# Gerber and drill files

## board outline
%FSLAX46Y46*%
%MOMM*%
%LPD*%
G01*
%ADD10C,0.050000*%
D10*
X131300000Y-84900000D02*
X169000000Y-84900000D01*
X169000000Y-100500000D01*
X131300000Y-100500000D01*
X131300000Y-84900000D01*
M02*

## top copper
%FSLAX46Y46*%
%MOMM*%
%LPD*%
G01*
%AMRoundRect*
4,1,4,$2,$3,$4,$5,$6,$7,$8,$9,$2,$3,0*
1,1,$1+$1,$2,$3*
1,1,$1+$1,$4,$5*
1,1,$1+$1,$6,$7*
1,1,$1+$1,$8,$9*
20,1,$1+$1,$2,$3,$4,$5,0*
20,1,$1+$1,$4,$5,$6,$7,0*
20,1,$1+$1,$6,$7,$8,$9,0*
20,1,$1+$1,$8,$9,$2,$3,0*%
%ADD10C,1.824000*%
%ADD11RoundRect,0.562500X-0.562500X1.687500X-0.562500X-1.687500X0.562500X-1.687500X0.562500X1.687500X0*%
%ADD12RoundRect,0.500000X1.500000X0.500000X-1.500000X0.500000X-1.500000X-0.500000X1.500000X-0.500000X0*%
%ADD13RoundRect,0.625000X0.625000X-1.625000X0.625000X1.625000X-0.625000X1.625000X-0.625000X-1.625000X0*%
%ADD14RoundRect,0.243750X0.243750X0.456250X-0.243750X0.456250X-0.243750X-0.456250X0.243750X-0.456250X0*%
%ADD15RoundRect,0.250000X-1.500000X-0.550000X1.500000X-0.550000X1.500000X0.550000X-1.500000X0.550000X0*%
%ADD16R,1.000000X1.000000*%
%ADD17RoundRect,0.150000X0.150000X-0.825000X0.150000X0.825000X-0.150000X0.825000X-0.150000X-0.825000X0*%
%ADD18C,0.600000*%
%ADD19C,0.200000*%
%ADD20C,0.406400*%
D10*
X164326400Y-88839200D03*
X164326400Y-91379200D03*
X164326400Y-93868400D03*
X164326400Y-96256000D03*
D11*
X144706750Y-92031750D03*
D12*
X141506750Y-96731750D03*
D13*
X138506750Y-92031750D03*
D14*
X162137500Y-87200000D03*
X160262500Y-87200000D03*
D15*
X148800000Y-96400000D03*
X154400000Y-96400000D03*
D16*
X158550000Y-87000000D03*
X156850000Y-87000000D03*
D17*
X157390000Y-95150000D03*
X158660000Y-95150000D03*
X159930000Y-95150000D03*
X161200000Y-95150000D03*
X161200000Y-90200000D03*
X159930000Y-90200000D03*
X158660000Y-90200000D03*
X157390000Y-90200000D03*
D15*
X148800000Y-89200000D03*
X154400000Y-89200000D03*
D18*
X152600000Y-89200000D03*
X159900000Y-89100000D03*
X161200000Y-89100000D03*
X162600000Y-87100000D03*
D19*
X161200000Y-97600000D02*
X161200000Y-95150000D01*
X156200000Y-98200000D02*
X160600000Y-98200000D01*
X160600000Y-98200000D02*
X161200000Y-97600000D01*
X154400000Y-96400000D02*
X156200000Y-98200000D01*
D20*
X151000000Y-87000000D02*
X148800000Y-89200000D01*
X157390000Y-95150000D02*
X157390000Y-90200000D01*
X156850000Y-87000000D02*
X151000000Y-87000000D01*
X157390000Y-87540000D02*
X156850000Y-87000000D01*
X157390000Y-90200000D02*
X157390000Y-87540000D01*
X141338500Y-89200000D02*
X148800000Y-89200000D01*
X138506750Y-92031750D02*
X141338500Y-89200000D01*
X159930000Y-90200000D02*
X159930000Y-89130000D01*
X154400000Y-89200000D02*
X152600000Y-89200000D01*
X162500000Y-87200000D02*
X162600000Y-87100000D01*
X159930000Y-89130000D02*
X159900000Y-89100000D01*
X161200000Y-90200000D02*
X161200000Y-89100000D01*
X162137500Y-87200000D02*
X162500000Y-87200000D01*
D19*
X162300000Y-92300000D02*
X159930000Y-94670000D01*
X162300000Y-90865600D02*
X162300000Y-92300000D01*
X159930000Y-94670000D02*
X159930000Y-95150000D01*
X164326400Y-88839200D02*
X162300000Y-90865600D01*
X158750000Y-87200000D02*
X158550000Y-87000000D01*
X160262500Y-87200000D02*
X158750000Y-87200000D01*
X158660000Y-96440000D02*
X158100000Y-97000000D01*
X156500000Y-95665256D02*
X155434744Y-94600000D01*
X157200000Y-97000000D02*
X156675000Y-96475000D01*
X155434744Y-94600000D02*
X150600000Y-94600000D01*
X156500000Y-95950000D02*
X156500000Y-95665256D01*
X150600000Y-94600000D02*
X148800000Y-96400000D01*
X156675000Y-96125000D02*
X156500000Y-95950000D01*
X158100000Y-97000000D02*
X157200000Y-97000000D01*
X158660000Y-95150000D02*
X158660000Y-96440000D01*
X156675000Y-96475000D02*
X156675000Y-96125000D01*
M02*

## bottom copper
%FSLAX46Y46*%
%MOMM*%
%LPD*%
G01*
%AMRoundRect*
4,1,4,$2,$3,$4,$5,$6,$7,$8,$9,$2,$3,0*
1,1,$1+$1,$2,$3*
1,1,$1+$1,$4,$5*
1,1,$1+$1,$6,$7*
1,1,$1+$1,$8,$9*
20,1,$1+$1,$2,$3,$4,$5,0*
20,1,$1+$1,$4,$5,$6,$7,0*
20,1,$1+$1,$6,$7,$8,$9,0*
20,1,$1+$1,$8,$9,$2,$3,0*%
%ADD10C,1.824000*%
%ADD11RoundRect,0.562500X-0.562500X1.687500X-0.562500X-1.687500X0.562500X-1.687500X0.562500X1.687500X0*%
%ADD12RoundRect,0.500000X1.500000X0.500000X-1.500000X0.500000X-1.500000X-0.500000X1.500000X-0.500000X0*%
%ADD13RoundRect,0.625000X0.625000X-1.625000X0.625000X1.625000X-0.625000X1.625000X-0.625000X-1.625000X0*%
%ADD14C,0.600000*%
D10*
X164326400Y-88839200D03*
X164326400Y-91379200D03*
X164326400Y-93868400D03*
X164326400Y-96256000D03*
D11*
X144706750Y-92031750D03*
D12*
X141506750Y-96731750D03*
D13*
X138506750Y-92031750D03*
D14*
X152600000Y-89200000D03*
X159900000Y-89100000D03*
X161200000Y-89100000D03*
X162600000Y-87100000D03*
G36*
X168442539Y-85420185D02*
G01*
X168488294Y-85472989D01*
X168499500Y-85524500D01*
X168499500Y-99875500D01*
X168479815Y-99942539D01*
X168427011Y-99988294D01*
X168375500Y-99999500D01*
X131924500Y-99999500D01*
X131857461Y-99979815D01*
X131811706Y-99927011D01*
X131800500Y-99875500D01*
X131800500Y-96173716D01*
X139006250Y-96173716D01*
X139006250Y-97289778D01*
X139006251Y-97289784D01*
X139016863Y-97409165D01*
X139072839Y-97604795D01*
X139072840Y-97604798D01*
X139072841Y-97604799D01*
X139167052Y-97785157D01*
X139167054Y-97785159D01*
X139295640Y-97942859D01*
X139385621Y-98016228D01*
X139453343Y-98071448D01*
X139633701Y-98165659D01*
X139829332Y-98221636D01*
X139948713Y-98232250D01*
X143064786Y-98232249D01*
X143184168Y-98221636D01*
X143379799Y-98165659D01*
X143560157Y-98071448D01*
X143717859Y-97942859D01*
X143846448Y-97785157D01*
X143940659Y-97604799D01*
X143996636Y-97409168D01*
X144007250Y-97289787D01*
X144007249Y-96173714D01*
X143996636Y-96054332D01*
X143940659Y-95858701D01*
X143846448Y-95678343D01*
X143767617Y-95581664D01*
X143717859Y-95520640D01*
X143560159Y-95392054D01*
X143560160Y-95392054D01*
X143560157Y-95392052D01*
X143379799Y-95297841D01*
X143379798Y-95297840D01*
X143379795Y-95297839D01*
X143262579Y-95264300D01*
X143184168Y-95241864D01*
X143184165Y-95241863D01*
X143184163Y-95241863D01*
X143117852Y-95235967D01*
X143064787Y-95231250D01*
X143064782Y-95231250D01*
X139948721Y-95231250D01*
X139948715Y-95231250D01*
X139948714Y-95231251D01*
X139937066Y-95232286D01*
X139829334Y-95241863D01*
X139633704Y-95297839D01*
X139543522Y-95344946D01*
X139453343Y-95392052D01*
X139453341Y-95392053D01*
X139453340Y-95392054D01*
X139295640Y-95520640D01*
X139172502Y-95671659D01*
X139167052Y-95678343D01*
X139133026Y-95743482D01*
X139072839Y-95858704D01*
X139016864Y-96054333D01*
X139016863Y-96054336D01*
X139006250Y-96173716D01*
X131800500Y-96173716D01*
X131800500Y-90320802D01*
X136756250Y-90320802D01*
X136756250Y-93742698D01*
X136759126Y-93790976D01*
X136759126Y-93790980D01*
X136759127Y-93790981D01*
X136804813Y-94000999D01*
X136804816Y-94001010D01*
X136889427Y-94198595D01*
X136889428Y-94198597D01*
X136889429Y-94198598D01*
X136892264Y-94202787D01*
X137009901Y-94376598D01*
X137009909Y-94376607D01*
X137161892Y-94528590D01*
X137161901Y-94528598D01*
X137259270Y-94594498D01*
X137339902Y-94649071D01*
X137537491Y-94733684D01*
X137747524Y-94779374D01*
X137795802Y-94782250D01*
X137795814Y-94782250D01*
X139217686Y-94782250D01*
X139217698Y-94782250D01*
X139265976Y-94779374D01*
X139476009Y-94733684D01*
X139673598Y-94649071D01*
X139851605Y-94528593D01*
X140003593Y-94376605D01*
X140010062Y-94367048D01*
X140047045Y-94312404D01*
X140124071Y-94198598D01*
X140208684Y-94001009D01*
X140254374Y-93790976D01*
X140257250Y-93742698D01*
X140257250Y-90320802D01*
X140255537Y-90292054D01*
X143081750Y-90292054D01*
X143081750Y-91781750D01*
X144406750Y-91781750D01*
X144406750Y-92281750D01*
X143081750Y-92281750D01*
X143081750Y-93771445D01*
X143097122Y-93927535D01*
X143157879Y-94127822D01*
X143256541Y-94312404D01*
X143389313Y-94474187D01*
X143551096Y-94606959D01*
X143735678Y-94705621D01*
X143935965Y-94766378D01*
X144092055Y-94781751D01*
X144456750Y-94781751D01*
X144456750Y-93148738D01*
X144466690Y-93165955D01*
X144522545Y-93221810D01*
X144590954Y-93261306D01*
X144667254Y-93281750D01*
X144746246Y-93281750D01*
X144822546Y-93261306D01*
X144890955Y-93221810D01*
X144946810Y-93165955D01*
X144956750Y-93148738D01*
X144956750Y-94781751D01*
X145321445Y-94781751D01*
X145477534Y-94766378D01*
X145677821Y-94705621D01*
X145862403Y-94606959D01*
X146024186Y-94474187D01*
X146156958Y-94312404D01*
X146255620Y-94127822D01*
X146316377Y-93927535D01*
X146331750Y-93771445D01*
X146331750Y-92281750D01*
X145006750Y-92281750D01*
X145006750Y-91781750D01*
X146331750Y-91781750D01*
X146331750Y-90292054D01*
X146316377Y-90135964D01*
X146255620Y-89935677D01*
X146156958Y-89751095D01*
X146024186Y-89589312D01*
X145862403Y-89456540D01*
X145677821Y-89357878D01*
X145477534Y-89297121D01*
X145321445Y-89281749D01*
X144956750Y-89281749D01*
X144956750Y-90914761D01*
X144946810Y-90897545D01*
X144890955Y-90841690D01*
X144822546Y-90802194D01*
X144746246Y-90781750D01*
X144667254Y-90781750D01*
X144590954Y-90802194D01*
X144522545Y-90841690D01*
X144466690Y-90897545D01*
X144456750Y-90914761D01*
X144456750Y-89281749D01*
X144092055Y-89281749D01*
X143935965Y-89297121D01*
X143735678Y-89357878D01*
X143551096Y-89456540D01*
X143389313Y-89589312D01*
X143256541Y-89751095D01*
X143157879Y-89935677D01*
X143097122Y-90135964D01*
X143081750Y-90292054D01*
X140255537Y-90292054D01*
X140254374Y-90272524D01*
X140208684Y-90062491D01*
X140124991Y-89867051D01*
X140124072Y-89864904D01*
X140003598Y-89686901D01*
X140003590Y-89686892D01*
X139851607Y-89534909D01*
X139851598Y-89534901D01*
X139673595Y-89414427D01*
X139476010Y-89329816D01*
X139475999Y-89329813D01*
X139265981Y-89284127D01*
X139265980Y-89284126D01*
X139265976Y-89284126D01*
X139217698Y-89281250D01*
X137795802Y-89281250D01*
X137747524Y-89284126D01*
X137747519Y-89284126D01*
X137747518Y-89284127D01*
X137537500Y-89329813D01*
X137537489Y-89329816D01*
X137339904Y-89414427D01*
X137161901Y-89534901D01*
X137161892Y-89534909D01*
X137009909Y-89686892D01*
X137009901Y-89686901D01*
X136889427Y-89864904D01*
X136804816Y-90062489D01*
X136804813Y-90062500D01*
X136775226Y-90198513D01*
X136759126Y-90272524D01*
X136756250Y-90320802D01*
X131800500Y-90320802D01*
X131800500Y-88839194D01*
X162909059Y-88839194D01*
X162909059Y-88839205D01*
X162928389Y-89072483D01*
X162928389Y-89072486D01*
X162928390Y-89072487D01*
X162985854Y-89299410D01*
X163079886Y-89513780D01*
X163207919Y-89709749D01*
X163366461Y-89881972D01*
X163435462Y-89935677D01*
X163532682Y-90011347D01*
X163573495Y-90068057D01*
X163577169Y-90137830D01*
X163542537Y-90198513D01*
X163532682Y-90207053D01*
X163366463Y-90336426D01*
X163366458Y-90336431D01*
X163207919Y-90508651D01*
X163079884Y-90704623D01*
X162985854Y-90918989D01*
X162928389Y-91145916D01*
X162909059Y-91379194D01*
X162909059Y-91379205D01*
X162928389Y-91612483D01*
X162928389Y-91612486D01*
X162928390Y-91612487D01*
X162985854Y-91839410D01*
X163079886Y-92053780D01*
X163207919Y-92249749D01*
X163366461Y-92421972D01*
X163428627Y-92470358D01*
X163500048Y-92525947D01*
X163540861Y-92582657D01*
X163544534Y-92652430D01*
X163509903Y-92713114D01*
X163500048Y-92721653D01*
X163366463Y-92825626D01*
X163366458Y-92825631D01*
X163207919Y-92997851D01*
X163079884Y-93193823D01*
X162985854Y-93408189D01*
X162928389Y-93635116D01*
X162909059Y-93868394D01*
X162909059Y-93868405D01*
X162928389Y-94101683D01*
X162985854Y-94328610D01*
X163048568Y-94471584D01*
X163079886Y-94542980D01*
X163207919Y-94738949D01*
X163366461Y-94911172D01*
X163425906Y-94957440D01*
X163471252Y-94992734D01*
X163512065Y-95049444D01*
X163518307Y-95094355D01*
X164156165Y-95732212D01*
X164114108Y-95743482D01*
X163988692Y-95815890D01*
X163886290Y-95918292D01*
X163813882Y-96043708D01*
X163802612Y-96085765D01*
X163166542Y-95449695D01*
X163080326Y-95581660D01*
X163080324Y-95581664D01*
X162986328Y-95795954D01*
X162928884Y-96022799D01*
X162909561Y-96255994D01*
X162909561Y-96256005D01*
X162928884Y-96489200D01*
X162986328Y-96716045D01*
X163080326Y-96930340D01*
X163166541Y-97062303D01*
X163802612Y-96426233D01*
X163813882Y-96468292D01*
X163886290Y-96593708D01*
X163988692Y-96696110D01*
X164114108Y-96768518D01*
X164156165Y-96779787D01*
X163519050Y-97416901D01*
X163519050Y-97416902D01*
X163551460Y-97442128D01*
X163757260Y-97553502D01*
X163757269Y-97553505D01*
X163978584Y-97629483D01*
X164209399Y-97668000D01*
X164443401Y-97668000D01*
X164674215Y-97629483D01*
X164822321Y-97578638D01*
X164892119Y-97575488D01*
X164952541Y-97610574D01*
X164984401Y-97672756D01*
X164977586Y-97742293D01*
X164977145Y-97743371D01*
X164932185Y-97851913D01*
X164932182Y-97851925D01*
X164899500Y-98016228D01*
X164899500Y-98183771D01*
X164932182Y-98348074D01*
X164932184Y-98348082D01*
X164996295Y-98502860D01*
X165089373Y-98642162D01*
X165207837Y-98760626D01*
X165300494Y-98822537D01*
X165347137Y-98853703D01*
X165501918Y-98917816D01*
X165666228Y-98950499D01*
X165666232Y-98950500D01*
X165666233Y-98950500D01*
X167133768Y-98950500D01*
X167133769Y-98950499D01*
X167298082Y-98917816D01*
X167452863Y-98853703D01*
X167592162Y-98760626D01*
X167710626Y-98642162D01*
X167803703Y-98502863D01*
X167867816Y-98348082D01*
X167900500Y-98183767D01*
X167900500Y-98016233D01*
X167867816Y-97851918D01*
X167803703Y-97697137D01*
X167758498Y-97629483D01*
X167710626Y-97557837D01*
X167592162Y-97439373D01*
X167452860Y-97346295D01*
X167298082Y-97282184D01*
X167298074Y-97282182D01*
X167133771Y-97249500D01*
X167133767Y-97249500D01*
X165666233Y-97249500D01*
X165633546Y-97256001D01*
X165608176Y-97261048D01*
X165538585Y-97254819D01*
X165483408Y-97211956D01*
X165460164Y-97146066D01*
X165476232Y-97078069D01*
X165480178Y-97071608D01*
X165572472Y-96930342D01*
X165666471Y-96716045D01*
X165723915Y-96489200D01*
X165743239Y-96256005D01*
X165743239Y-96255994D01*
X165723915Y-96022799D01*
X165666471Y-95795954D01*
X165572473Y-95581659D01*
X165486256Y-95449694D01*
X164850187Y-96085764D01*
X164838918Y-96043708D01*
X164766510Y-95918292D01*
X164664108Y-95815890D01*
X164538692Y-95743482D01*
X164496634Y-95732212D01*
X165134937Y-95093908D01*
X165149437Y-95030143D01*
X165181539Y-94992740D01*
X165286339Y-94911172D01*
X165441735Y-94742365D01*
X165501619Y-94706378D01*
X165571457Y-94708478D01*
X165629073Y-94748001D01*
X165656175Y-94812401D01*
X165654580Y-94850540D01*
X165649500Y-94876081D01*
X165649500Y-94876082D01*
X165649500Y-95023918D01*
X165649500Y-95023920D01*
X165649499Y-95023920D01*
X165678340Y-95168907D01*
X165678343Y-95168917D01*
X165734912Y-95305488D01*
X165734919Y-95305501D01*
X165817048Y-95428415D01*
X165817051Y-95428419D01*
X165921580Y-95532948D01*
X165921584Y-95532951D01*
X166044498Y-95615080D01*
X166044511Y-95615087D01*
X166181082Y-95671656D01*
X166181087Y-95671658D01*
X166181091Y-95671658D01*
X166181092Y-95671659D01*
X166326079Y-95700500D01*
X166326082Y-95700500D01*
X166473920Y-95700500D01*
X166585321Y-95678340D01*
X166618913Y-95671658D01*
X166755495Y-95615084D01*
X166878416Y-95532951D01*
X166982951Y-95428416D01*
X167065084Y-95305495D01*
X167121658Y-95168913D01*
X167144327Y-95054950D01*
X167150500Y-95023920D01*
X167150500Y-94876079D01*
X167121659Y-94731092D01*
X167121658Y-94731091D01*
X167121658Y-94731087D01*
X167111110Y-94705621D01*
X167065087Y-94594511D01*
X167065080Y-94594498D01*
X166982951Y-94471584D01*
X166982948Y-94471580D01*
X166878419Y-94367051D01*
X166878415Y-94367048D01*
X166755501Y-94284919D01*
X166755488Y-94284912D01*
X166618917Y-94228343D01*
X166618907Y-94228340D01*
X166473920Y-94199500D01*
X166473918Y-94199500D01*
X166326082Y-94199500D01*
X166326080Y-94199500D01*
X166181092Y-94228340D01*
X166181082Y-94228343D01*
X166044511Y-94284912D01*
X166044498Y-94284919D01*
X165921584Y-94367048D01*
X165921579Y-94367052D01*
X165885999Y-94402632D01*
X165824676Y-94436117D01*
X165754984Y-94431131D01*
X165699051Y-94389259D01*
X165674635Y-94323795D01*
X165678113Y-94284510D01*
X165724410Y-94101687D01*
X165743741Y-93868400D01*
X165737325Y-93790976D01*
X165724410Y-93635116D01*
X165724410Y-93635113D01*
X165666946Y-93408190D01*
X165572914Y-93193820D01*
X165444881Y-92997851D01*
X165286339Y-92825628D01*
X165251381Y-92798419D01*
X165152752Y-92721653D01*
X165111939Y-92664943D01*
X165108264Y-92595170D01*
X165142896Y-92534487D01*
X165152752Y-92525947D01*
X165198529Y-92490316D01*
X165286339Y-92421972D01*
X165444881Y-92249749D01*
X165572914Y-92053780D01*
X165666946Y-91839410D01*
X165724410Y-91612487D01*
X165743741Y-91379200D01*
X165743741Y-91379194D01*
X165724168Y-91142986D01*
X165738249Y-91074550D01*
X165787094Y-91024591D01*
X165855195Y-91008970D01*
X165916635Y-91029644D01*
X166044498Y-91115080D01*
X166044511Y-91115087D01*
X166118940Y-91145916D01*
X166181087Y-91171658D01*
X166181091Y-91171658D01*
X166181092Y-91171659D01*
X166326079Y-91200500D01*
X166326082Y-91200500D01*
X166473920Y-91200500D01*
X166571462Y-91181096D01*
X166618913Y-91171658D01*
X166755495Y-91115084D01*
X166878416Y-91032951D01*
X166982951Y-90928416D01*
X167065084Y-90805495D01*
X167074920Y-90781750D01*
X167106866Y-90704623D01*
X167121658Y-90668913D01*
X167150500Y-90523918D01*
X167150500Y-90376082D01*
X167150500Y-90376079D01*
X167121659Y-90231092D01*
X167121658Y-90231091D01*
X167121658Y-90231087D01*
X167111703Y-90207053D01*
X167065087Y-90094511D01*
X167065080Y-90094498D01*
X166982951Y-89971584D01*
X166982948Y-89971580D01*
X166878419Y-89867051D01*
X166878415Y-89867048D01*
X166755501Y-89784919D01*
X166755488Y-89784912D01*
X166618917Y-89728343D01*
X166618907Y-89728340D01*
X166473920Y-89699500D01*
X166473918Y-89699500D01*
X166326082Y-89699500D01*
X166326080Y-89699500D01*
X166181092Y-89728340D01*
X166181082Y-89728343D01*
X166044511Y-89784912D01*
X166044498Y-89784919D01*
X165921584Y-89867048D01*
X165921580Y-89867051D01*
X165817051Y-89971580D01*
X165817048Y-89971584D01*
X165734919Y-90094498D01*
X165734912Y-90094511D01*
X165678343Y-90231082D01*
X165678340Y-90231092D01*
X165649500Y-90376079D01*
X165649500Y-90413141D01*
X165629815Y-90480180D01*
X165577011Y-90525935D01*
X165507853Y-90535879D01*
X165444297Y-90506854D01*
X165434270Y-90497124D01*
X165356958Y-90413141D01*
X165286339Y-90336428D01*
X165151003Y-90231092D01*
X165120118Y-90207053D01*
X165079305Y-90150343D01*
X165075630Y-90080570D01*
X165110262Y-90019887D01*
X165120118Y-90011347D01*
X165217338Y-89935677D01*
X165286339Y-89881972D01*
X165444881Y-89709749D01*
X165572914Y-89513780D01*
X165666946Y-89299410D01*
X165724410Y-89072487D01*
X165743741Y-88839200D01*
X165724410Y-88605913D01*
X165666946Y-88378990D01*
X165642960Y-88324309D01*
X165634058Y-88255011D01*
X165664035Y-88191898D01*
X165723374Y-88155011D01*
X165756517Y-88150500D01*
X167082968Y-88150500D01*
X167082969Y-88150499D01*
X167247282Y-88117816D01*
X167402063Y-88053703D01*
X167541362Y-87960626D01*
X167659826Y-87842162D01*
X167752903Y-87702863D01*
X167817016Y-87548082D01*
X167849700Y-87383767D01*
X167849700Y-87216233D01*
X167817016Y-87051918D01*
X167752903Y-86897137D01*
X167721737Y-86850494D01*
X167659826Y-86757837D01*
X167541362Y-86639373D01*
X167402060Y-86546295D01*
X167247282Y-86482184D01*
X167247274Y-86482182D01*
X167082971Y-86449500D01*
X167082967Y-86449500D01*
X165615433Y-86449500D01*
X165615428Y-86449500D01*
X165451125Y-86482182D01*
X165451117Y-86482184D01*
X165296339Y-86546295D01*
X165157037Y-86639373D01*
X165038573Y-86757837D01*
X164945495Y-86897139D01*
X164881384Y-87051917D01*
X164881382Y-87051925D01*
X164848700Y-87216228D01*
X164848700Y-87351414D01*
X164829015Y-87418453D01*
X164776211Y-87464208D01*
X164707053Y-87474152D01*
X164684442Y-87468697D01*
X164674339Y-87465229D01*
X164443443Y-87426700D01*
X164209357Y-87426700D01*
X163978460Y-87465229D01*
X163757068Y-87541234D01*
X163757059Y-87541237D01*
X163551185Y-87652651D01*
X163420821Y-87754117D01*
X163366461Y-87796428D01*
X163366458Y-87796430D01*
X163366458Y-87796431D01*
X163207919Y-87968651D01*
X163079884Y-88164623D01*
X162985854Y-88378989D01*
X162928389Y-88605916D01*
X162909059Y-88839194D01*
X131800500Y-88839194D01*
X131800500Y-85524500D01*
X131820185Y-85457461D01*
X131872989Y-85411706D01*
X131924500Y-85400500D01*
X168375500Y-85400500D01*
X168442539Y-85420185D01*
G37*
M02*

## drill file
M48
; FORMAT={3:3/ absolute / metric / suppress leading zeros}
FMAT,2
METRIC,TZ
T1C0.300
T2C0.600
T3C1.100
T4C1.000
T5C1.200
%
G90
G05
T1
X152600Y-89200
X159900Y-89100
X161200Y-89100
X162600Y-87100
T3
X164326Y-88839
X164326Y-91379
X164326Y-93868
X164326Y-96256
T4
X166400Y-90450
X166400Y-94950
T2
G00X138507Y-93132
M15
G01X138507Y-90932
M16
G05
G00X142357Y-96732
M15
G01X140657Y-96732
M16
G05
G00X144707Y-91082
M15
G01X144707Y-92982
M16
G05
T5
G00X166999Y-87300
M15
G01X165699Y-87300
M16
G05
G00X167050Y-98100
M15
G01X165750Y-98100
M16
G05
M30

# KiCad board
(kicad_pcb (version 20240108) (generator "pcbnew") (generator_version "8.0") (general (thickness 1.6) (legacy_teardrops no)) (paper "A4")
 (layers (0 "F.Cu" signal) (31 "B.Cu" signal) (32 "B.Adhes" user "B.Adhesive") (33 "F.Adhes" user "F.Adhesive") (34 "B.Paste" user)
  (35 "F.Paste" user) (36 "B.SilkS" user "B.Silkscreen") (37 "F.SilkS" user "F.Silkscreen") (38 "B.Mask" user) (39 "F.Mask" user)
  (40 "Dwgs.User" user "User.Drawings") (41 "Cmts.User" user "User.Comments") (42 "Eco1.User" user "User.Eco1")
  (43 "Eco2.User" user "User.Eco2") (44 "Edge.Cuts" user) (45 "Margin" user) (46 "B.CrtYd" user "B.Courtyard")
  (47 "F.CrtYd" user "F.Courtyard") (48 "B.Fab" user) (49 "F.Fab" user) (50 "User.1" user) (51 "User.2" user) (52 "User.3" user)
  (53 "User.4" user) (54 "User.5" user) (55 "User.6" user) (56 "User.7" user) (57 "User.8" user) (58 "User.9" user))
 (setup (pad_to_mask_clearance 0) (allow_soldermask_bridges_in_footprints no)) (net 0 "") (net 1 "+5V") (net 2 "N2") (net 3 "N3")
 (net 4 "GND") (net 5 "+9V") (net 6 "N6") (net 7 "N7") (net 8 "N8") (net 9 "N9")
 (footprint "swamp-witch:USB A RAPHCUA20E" (layer "F.Cu") (at 174.4264 92.7 180)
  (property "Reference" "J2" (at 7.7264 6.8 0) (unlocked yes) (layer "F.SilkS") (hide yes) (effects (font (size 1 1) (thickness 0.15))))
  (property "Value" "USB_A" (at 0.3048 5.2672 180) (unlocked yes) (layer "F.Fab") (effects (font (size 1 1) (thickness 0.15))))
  (pad "" np_thru_hole oval (at 8.0264 -5.4 180) (size 2.5 1.2) (drill oval 2.5 1.2) (layers "F&B.Cu" "*.Mask"))
  (pad "" np_thru_hole circle (at 8.0264 -2.25 180) (size 1 1) (drill 1) (layers "F&B.Cu" "*.Mask"))
  (pad "" np_thru_hole circle (at 8.0264 2.25 180) (size 1 1) (drill 1) (layers "F&B.Cu" "*.Mask"))
  (pad "" np_thru_hole oval (at 8.0772 5.4 180) (size 2.5 1.2) (drill oval 2.5 1.2) (layers "F&B.Cu" "*.Mask"))
  (pad "1" thru_hole circle (at 10.1 3.8608 180) (size 1.824 1.824) (drill 1.1) (layers "*.Cu" "*.Mask") (remove_unused_layers no)
   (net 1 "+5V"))
  (pad "2" thru_hole circle (at 10.1 1.3208 180) (size 1.824 1.824) (drill 1.1) (layers "*.Cu" "*.Mask") (remove_unused_layers no)
   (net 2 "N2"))
  (pad "3" thru_hole circle (at 10.1 -1.1684 180) (size 1.824 1.824) (drill 1.1) (layers "*.Cu" "*.Mask") (remove_unused_layers no)
   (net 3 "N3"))
  (pad "4" thru_hole circle (at 10.1 -3.556 180) (size 1.824 1.824) (drill 1.1) (layers "*.Cu" "*.Mask") (remove_unused_layers no)
   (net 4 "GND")))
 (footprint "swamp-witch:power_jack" (layer "F.Cu") (at 138.05675 92.03175 180)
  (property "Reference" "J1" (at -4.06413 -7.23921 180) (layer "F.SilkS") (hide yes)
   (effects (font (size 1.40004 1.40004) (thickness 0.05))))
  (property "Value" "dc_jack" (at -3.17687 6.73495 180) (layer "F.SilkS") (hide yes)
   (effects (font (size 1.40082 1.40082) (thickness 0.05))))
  (pad "1" thru_hole roundrect (at -6.65 0 270) (size 4.500001 2.25) (drill oval 2.5 0.6) (layers "*.Cu" "*.Mask") (remove_unused_layers no)
   (roundrect_rratio 0.25) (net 4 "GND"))
  (pad "2" thru_hole roundrect (at -3.45 -4.7 180) (size 4 2) (drill oval 2.3 0.6) (layers "*.Cu" "*.Mask") (remove_unused_layers no)
   (roundrect_rratio 0.25))
  (pad "3" thru_hole roundrect (at -0.45 0 90) (size 4.5 2.5) (drill oval 2.8 0.6) (layers "*.Cu" "*.Mask") (remove_unused_layers no)
   (roundrect_rratio 0.25) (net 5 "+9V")))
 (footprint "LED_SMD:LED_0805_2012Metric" (layer "F.Cu") (at 161.2 87.2 180)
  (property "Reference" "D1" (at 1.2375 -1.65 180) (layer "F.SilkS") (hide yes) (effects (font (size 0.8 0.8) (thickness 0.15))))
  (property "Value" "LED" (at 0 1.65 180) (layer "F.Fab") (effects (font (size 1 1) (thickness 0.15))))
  (pad "1" smd roundrect (at -0.9375 0 180) (size 0.975 1.4) (layers "F.Cu" "F.Paste" "F.Mask") (roundrect_rratio 0.25) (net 4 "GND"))
  (pad "2" smd roundrect (at 0.9375 0 180) (size 0.975 1.4) (layers "F.Cu" "F.Paste" "F.Mask") (roundrect_rratio 0.25) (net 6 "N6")))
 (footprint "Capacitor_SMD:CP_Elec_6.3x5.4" (layer "F.Cu") (at 151.6 96.4)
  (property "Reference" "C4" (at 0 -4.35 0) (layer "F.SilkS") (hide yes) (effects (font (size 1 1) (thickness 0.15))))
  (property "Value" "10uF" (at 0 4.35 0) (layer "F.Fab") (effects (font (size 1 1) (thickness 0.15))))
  (pad "1" smd roundrect (at -2.8 0) (size 3.5 1.6) (layers "F.Cu" "F.Paste" "F.Mask") (roundrect_rratio 0.15625) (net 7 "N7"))
  (pad "2" smd roundrect (at 2.8 0) (size 3.5 1.6) (layers "F.Cu" "F.Paste" "F.Mask") (roundrect_rratio 0.15625) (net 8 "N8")))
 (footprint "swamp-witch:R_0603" (layer "F.Cu") (at 157.7 87 180)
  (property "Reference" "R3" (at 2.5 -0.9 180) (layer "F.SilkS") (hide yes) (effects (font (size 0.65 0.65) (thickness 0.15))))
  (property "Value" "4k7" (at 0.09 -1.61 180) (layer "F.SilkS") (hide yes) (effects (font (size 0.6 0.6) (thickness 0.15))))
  (pad "1" smd rect (at -0.85 0 180) (size 1 1) (layers "F.Cu" "F.Paste" "F.Mask") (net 6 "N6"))
  (pad "2" smd rect (at 0.85 0 180) (size 1 1) (layers "F.Cu" "F.Paste" "F.Mask") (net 5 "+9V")))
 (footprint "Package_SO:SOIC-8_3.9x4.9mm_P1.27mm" (layer "F.Cu") (at 159.295 92.675 90)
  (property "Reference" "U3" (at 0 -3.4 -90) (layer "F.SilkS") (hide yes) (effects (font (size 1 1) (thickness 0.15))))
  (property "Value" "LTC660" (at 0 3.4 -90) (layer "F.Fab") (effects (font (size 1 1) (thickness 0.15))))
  (pad "1" smd roundrect (at -2.475 -1.905 90) (size 1.95 0.6) (layers "F.Cu" "F.Paste" "F.Mask") (roundrect_rratio 0.25) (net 5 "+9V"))
  (pad "2" smd roundrect (at -2.475 -0.635 90) (size 1.95 0.6) (layers "F.Cu" "F.Paste" "F.Mask") (roundrect_rratio 0.25) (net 7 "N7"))
  (pad "3" smd roundrect (at -2.475 0.635 90) (size 1.95 0.6) (layers "F.Cu" "F.Paste" "F.Mask") (roundrect_rratio 0.25) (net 1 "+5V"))
  (pad "4" smd roundrect (at -2.475 1.905 90) (size 1.95 0.6) (layers "F.Cu" "F.Paste" "F.Mask") (roundrect_rratio 0.25) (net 8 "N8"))
  (pad "5" smd roundrect (at 2.475 1.905 90) (size 1.95 0.6) (layers "F.Cu" "F.Paste" "F.Mask") (roundrect_rratio 0.25) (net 4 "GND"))
  (pad "6" smd roundrect (at 2.475 0.635 90) (size 1.95 0.6) (layers "F.Cu" "F.Paste" "F.Mask") (roundrect_rratio 0.25) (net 4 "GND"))
  (pad "7" smd roundrect (at 2.475 -0.635 90) (size 1.95 0.6) (layers "F.Cu" "F.Paste" "F.Mask") (roundrect_rratio 0.25) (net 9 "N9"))
  (pad "8" smd roundrect (at 2.475 -1.905 90) (size 1.95 0.6) (layers "F.Cu" "F.Paste" "F.Mask") (roundrect_rratio 0.25) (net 5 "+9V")))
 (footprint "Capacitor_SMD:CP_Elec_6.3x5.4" (layer "F.Cu") (at 151.6 89.2)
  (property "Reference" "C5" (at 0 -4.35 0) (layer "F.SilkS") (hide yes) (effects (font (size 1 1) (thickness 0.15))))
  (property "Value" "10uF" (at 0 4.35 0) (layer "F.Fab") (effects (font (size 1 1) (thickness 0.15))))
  (pad "1" smd roundrect (at -2.8 0) (size 3.5 1.6) (layers "F.Cu" "F.Paste" "F.Mask") (roundrect_rratio 0.15625) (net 5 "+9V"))
  (pad "2" smd roundrect (at 2.8 0) (size 3.5 1.6) (layers "F.Cu" "F.Paste" "F.Mask") (roundrect_rratio 0.15625) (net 4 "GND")))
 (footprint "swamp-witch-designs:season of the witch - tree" (layer "B.Cu") (at 143.05 93.59 90)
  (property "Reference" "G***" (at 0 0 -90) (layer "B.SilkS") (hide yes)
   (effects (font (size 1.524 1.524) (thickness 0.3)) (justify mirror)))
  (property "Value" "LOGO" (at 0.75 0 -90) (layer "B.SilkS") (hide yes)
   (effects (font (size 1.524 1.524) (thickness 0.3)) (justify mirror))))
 (gr_rect (start 131.3 84.9) (end 169 100.5) (stroke (width 0.05) (type default)) (fill none) (layer "Edge.Cuts"))
 (segment (start 161.2 97.6) (end 161.2 95.15) (width 0.2) (layer "F.Cu") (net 8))
 (segment (start 156.2 98.2) (end 160.6 98.2) (width 0.2) (layer "F.Cu") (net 8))
 (segment (start 160.6 98.2) (end 161.2 97.6) (width 0.2) (layer "F.Cu") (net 8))
 (segment (start 154.4 96.4) (end 156.2 98.2) (width 0.2) (layer "F.Cu") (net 8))
 (segment (start 151 87) (end 148.8 89.2) (width 0.4064) (layer "F.Cu") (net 5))
 (segment (start 157.39 95.15) (end 157.39 90.2) (width 0.4064) (layer "F.Cu") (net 5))
 (segment (start 156.85 87) (end 151 87) (width 0.4064) (layer "F.Cu") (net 5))
 (segment (start 157.39 87.54) (end 156.85 87) (width 0.4064) (layer "F.Cu") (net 5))
 (segment (start 157.39 90.2) (end 157.39 87.54) (width 0.4064) (layer "F.Cu") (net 5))
 (segment (start 141.3385 89.2) (end 148.8 89.2) (width 0.4064) (layer "F.Cu") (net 5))
 (segment (start 138.50675 92.03175) (end 141.3385 89.2) (width 0.4064) (layer "F.Cu") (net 5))
 (segment (start 159.93 90.2) (end 159.93 89.13) (width 0.4064) (layer "F.Cu") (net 4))
 (segment (start 154.4 89.2) (end 152.6 89.2) (width 0.4064) (layer "F.Cu") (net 4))
 (segment (start 162.5 87.2) (end 162.6 87.1) (width 0.4064) (layer "F.Cu") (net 4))
 (segment (start 159.93 89.13) (end 159.9 89.1) (width 0.4064) (layer "F.Cu") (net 4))
 (segment (start 161.2 90.2) (end 161.2 89.1) (width 0.4064) (layer "F.Cu") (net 4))
 (segment (start 162.1375 87.2) (end 162.5 87.2) (width 0.4064) (layer "F.Cu") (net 4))
 (via (at 152.6 89.2) (size 0.6) (drill 0.3) (layers "F.Cu" "B.Cu") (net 4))
 (via (at 159.9 89.1) (size 0.6) (drill 0.3) (layers "F.Cu" "B.Cu") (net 4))
 (via (at 161.2 89.1) (size 0.6) (drill 0.3) (layers "F.Cu" "B.Cu") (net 4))
 (via (at 162.6 87.1) (size 0.6) (drill 0.3) (layers "F.Cu" "B.Cu") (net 4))
 (segment (start 162.3 92.3) (end 159.93 94.67) (width 0.2) (layer "F.Cu") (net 1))
 (segment (start 162.3 90.8656) (end 162.3 92.3) (width 0.2) (layer "F.Cu") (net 1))
 (segment (start 159.93 94.67) (end 159.93 95.15) (width 0.2) (layer "F.Cu") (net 1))
 (segment (start 164.3264 88.8392) (end 162.3 90.8656) (width 0.2) (layer "F.Cu") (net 1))
 (segment (start 158.75 87.2) (end 158.55 87) (width 0.2) (layer "F.Cu") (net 6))
 (segment (start 160.2625 87.2) (end 158.75 87.2) (width 0.2) (layer "F.Cu") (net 6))
 (segment (start 158.66 96.44) (end 158.1 97) (width 0.2) (layer "F.Cu") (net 7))
 (segment (start 156.5 95.665256) (end 155.434744 94.6) (width 0.2) (layer "F.Cu") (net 7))
 (segment (start 157.2 97) (end 156.675 96.475) (width 0.2) (layer "F.Cu") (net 7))
 (segment (start 155.434744 94.6) (end 150.6 94.6) (width 0.2) (layer "F.Cu") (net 7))
 (segment (start 156.5 95.95) (end 156.5 95.665256) (width 0.2) (layer "F.Cu") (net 7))
 (segment (start 150.6 94.6) (end 148.8 96.4) (width 0.2) (layer "F.Cu") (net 7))
 (segment (start 156.675 96.125) (end 156.5 95.95) (width 0.2) (layer "F.Cu") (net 7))
 (segment (start 158.1 97) (end 157.2 97) (width 0.2) (layer "F.Cu") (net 7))
 (segment (start 158.66 95.15) (end 158.66 96.44) (width 0.2) (layer "F.Cu") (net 7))
 (segment (start 156.675 96.475) (end 156.675 96.125) (width 0.2) (layer "F.Cu") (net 7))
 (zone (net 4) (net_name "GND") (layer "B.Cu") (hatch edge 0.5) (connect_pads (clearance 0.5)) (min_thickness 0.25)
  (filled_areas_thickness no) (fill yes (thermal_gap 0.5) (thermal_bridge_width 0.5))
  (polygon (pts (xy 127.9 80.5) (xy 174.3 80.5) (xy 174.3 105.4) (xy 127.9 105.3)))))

